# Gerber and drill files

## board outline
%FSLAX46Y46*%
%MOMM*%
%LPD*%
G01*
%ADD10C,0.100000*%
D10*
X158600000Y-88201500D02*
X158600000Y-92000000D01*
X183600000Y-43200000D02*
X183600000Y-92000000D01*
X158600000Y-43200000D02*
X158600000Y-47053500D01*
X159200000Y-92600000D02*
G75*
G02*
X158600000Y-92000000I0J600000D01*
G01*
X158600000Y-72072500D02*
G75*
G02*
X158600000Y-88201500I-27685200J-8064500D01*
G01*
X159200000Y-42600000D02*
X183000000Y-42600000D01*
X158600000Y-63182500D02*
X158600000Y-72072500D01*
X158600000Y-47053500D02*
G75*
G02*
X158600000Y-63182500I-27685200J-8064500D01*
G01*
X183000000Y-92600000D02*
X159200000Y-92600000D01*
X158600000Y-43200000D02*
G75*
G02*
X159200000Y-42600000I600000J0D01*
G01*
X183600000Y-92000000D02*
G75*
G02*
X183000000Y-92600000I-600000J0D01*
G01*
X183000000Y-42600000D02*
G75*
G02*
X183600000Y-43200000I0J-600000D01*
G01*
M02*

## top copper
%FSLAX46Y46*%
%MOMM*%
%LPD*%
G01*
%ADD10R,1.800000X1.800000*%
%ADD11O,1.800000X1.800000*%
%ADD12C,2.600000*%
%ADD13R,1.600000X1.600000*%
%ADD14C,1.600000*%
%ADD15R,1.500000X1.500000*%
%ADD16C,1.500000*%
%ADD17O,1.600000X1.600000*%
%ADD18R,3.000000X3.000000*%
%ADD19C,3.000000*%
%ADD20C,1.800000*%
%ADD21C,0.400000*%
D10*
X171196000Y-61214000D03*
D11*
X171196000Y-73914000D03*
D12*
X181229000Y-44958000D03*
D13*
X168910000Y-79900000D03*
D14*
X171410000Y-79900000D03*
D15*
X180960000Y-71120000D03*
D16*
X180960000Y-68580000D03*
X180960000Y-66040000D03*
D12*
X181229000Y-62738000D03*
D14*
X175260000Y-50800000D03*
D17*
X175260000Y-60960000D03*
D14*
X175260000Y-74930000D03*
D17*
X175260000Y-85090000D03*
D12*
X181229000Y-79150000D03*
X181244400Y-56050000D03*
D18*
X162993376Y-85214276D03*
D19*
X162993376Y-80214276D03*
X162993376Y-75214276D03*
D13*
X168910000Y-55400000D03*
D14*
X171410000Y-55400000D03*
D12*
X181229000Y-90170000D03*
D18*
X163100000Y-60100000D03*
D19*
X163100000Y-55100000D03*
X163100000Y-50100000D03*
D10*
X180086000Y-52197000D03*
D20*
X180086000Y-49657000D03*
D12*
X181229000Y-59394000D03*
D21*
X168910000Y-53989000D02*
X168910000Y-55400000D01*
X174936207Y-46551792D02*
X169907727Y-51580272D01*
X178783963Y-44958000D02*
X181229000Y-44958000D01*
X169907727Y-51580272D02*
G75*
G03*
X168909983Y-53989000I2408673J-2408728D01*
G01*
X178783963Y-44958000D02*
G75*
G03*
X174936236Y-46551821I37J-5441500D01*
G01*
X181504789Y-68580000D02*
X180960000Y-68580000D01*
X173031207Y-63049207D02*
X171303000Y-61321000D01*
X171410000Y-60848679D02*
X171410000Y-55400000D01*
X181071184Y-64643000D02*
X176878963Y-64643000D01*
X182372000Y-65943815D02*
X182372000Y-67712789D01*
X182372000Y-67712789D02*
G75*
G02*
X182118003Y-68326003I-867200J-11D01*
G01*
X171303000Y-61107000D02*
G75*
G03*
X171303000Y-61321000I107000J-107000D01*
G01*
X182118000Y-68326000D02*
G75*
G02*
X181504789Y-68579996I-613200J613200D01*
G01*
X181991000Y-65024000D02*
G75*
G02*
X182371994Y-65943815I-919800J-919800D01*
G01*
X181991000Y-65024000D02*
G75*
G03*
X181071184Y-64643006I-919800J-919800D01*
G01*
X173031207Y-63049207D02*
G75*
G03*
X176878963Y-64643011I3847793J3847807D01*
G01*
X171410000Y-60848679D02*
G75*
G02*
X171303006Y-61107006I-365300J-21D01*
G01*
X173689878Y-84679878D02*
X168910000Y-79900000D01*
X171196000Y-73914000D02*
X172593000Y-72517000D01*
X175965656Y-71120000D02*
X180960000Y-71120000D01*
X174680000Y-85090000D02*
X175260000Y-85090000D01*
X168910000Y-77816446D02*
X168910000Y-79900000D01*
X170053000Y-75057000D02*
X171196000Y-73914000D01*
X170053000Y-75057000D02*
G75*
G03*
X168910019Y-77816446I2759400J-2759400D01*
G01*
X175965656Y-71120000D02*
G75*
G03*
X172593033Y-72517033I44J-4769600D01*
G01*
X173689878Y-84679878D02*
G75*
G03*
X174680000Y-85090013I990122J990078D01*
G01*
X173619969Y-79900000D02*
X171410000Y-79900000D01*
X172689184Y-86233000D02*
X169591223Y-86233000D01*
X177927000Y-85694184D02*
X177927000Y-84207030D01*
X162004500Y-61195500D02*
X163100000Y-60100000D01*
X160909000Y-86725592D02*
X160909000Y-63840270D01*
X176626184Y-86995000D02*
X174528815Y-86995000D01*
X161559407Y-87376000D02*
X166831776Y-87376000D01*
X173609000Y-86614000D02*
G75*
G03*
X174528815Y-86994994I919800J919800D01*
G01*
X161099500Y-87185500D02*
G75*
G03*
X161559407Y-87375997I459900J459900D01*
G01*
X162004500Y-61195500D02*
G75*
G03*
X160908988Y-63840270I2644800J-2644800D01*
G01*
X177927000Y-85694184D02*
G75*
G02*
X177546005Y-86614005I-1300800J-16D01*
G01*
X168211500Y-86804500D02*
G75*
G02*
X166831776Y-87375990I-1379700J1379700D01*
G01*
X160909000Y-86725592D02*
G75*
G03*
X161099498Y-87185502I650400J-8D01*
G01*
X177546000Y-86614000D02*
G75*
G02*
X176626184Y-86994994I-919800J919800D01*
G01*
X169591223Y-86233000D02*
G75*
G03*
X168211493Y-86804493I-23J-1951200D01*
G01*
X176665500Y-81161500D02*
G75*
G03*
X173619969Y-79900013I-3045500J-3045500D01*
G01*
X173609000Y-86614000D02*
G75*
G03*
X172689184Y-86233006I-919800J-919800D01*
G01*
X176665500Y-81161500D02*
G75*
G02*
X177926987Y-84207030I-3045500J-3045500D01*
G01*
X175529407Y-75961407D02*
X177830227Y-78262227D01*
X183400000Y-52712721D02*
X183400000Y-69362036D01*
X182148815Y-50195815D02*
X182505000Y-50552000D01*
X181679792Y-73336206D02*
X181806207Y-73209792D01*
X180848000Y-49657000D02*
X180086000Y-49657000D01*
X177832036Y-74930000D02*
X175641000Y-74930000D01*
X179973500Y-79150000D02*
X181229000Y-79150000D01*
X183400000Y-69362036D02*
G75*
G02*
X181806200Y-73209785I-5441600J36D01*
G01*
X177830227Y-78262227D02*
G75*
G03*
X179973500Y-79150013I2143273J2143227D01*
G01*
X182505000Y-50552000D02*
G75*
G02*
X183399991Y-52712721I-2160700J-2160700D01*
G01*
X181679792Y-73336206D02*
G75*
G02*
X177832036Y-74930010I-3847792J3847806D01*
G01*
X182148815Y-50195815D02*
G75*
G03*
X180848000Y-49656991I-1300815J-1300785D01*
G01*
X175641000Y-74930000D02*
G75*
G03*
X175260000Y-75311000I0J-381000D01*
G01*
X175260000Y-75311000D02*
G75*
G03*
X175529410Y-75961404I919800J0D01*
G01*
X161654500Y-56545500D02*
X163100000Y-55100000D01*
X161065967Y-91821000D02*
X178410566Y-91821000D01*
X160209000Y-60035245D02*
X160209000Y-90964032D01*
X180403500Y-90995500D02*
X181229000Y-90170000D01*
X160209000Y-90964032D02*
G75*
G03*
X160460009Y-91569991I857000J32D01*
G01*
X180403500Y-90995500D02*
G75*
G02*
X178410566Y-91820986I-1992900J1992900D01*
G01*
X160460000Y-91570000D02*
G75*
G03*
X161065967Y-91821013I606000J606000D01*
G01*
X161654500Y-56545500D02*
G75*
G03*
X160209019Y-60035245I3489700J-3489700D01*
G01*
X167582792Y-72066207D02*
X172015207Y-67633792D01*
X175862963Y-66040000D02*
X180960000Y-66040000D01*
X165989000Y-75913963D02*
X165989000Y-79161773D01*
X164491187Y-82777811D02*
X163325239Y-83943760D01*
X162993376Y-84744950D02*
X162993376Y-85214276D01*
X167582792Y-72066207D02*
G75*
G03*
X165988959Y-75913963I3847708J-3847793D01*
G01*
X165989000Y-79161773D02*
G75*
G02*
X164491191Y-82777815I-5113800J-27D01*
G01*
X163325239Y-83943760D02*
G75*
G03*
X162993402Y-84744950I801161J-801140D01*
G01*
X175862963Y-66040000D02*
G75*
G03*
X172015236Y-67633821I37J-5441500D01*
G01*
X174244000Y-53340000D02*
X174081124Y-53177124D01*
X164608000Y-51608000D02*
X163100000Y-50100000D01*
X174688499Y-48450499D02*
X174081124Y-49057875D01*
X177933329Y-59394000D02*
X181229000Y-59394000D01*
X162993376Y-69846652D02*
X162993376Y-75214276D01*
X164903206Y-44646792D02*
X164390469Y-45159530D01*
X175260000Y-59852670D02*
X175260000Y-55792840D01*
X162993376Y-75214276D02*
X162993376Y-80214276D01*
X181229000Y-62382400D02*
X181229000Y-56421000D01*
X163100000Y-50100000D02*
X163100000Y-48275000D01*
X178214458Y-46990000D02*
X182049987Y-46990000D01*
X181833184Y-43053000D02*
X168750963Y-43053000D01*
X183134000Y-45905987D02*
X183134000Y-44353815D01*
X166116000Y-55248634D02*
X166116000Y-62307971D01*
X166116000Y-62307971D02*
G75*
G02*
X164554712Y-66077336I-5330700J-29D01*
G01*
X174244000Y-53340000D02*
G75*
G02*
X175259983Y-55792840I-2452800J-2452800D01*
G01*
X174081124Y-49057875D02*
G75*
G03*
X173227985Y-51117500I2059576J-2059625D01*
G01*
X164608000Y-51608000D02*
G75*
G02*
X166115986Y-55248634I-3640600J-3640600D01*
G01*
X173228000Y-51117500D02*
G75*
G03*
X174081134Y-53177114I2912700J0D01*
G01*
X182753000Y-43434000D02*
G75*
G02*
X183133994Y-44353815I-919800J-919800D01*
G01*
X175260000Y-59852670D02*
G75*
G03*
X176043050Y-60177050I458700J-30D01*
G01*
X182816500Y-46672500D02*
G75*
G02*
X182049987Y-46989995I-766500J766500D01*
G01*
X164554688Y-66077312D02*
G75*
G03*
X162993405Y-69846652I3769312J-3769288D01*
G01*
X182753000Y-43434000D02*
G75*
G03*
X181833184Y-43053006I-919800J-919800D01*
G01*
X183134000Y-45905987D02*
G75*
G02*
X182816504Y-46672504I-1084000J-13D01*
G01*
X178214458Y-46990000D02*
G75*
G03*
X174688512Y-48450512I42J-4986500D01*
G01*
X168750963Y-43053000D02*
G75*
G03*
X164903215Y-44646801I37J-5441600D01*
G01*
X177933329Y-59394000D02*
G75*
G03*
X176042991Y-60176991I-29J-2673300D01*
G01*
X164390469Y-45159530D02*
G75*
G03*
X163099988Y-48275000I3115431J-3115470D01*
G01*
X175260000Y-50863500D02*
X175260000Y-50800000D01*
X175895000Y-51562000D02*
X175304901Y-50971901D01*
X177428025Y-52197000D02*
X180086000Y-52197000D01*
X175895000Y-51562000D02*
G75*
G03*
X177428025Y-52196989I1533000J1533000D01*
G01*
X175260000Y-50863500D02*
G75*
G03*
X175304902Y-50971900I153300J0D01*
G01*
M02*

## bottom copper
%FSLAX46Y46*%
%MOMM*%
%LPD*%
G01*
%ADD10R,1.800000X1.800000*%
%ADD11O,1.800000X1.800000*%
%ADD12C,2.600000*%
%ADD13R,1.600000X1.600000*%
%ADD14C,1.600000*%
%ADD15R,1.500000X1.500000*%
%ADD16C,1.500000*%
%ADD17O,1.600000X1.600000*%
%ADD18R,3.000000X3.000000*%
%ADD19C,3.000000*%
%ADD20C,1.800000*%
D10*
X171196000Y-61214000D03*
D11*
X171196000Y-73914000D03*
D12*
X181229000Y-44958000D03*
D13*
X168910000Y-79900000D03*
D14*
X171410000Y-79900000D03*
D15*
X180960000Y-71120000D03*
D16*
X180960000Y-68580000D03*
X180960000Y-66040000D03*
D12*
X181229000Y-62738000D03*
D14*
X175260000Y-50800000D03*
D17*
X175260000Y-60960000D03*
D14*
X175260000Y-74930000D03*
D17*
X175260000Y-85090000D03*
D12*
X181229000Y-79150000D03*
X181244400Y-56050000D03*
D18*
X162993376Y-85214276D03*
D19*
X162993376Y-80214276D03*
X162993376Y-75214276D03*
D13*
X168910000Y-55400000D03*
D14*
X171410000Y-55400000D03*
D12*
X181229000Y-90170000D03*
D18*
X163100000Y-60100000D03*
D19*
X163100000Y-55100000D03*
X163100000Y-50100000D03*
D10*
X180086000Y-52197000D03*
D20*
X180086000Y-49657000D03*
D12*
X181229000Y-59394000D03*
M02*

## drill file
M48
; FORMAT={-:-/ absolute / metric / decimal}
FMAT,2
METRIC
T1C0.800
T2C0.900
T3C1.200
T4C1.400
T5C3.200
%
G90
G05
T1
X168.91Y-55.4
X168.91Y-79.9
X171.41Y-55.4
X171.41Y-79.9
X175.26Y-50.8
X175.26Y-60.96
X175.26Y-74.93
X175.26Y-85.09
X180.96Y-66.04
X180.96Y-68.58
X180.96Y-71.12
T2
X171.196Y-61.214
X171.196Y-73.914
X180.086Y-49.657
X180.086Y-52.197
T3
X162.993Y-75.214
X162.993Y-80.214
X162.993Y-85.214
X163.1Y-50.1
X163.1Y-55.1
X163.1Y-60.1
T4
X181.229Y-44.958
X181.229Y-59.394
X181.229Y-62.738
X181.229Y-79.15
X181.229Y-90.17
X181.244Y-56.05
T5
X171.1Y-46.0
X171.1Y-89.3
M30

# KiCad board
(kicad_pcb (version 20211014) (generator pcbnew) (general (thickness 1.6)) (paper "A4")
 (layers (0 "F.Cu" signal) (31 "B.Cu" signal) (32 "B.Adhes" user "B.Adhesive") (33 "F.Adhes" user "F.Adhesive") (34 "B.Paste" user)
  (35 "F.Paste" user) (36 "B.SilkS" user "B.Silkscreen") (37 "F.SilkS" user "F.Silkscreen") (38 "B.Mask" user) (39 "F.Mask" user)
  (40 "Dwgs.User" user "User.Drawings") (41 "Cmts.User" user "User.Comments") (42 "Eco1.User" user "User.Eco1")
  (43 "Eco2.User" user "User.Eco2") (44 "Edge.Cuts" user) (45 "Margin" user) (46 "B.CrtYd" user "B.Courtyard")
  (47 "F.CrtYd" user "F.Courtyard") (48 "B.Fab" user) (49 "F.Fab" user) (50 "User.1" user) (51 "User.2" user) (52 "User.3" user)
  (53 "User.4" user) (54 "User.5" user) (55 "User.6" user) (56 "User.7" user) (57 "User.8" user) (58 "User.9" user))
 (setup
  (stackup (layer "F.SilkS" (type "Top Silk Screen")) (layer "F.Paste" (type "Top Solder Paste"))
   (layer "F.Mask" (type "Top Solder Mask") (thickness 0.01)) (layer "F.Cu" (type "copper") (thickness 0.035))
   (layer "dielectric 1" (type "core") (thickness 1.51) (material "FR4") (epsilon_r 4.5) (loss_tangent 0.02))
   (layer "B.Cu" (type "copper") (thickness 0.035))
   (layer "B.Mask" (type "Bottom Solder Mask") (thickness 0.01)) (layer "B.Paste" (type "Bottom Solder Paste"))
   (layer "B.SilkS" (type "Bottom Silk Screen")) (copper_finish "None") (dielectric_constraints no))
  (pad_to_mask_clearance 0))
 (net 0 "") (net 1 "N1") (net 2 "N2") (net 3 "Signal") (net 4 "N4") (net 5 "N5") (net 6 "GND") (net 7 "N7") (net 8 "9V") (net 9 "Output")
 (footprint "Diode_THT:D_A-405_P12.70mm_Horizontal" (layer "F.Cu") (at 171.196 61.214 -90)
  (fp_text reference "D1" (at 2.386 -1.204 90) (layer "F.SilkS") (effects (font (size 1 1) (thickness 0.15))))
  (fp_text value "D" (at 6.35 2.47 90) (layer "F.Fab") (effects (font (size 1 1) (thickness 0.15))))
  (pad "1" thru_hole rect (at 0 0 270) (size 1.8 1.8) (drill 0.9) (layers *.Cu *.Mask) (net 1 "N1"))
  (pad "2" thru_hole oval (at 12.7 0 270) (size 1.8 1.8) (drill 0.9) (layers *.Cu *.Mask) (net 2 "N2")))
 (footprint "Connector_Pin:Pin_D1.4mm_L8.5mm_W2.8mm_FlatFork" (layer "F.Cu") (at 181.229 44.958)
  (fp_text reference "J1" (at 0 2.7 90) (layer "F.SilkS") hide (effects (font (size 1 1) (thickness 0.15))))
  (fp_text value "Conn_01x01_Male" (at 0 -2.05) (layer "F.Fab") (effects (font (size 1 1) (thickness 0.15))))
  (pad "1" thru_hole circle (at 0 0) (size 2.6 2.6) (drill 1.4) (layers *.Cu *.Mask) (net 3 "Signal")))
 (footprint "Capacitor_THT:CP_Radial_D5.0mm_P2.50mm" (layer "F.Cu") (at 168.91 79.9)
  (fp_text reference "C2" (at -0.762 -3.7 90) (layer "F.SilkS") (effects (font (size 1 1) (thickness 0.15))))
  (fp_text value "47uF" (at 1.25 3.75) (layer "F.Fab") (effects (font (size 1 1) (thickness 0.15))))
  (pad "1" thru_hole rect (at 0 0) (size 1.6 1.6) (drill 0.8) (layers *.Cu *.Mask) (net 2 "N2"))
  (pad "2" thru_hole circle (at 2.5 0) (size 1.6 1.6) (drill 0.8) (layers *.Cu *.Mask) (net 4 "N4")))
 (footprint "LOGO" (layer "F.Cu") (at 164.214424 67.737512 90)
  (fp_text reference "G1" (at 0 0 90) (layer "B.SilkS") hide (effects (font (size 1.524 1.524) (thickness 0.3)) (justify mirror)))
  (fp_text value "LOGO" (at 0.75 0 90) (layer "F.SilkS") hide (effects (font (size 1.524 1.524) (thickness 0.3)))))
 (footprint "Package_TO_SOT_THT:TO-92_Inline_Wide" (layer "F.Cu") (at 180.96 71.12 90)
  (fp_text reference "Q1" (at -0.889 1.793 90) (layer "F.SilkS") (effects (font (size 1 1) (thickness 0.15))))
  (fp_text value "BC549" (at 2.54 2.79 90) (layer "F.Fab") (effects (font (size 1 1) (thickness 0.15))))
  (pad "1" thru_hole rect (at 0 0 90) (size 1.5 1.5) (drill 0.8) (layers *.Cu *.Mask) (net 2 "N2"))
  (pad "2" thru_hole circle (at 2.54 0 90) (size 1.5 1.5) (drill 0.8) (layers *.Cu *.Mask) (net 1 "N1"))
  (pad "3" thru_hole circle (at 5.08 0 90) (size 1.5 1.5) (drill 0.8) (layers *.Cu *.Mask) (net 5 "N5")))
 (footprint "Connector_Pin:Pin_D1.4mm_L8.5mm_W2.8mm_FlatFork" (layer "F.Cu") (at 181.229 62.738)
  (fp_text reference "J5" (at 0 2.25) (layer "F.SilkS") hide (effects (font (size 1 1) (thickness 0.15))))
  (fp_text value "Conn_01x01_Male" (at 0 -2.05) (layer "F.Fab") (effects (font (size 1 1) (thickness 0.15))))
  (pad "1" thru_hole circle (at 0 0) (size 2.6 2.6) (drill 1.4) (layers *.Cu *.Mask) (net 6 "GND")))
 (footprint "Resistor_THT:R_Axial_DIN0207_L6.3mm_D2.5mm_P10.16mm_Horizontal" (layer "F.Cu") (at 175.26 50.8 -90)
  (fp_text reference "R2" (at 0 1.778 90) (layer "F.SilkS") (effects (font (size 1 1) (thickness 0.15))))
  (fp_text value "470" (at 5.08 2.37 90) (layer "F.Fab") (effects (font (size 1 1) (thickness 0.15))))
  (pad "1" thru_hole circle (at 0 0 270) (size 1.6 1.6) (drill 0.8) (layers *.Cu *.Mask) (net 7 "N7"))
  (pad "2" thru_hole oval (at 10.16 0 270) (size 1.6 1.6) (drill 0.8) (layers *.Cu *.Mask) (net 6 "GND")))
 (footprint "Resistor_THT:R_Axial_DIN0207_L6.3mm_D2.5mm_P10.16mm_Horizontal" (layer "F.Cu") (at 175.26 74.93 -90)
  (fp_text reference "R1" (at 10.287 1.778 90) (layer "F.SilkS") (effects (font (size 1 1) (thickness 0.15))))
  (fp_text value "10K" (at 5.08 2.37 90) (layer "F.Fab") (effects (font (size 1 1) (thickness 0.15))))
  (pad "1" thru_hole circle (at 0 0 270) (size 1.6 1.6) (drill 0.8) (layers *.Cu *.Mask) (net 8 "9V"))
  (pad "2" thru_hole oval (at 10.16 0 270) (size 1.6 1.6) (drill 0.8) (layers *.Cu *.Mask) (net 2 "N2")))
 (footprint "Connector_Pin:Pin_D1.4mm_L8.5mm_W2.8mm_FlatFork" (layer "F.Cu") (at 181.229 79.15)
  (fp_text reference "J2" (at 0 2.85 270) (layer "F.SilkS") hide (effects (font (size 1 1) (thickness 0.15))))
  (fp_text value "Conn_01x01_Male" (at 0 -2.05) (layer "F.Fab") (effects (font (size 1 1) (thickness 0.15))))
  (pad "1" thru_hole circle (at 0 0) (size 2.6 2.6) (drill 1.4) (layers *.Cu *.Mask) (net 8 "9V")))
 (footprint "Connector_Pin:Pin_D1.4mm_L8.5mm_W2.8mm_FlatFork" (layer "F.Cu") (at 181.2444 56.05)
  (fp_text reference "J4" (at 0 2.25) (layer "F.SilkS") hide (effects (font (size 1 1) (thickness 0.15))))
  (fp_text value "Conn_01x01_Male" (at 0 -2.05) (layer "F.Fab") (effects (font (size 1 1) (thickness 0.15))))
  (pad "1" thru_hole circle (at 0 0) (size 2.6 2.6) (drill 1.4) (layers *.Cu *.Mask) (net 6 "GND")))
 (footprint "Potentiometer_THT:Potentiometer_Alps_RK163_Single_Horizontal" (layer "F.Cu") (at 162.7775 79.996 180)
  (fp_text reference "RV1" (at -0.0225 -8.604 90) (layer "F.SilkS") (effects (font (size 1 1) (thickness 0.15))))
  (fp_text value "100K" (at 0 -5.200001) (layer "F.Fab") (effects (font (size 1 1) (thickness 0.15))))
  (pad "1" thru_hole rect (at -0.215876 -5.218276) (size 3 3) (drill 1.2) (layers *.Cu *.Mask) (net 5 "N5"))
  (pad "2" thru_hole circle (at -0.215876 -0.218276) (size 3 3) (drill 1.2) (layers *.Cu *.Mask) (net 6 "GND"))
  (pad "3" thru_hole circle (at -0.215876 4.781724) (size 3 3) (drill 1.2) (layers *.Cu *.Mask) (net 6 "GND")))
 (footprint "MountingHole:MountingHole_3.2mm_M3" (layer "F.Cu") (at 171.1 46)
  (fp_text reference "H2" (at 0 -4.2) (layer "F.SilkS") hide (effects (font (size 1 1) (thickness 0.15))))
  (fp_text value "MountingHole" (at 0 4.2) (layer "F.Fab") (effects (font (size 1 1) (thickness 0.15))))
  (pad "" np_thru_hole circle (at 0 0) (size 3.2 3.2) (drill 3.2) (layers *.Cu *.Mask)))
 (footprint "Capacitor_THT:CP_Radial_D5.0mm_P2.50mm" (layer "F.Cu") (at 168.91 55.4)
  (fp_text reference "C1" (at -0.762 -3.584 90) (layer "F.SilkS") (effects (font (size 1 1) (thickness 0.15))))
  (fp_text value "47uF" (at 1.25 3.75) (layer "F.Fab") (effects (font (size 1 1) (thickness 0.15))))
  (pad "1" thru_hole rect (at 0 0) (size 1.6 1.6) (drill 0.8) (layers *.Cu *.Mask) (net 3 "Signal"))
  (pad "2" thru_hole circle (at 2.5 0) (size 1.6 1.6) (drill 0.8) (layers *.Cu *.Mask) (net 1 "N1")))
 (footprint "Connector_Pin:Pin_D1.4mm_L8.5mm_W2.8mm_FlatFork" (layer "F.Cu") (at 181.229 90.17)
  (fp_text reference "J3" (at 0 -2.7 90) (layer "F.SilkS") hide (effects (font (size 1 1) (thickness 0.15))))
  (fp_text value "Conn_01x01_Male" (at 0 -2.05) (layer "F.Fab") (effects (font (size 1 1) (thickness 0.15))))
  (pad "1" thru_hole circle (at 0 0) (size 2.6 2.6) (drill 1.4) (layers *.Cu *.Mask) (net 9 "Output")))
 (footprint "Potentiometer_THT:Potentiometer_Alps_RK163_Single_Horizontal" (layer "F.Cu") (at 163.1 60.1 180)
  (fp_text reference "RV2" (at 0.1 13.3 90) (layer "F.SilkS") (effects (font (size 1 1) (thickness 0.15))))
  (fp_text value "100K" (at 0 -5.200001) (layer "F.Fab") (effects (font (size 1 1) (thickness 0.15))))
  (pad "1" thru_hole rect (at 0 0) (size 3 3) (drill 1.2) (layers *.Cu *.Mask) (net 4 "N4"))
  (pad "2" thru_hole circle (at 0 5) (size 3 3) (drill 1.2) (layers *.Cu *.Mask) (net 9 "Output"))
  (pad "3" thru_hole circle (at 0 10) (size 3 3) (drill 1.2) (layers *.Cu *.Mask) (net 6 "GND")))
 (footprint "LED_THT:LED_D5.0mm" (layer "F.Cu") (at 180.086 52.197 90)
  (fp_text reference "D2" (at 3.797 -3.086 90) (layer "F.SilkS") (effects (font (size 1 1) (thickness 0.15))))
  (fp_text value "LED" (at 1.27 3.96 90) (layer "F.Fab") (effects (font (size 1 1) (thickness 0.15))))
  (pad "1" thru_hole rect (at 0 0 90) (size 1.8 1.8) (drill 0.9) (layers *.Cu *.Mask) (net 7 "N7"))
  (pad "2" thru_hole circle (at 2.54 0 90) (size 1.8 1.8) (drill 0.9) (layers *.Cu *.Mask) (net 8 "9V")))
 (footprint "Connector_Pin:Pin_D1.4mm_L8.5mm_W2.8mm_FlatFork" (layer "F.Cu") (at 181.229 59.394 180)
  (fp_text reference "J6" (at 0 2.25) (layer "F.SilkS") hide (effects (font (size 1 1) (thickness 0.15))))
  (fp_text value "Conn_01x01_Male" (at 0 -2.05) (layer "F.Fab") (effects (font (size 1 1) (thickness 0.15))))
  (pad "1" thru_hole circle (at 0 0 180) (size 2.6 2.6) (drill 1.4) (layers *.Cu *.Mask) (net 6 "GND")))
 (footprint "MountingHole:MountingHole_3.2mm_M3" (layer "F.Cu") (at 171.1 89.3)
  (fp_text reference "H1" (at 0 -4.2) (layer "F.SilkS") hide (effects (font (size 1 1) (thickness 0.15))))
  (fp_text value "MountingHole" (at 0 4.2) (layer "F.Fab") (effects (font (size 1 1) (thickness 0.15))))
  (pad "" np_thru_hole circle (at 0 0) (size 3.2 3.2) (drill 3.2) (layers *.Cu *.Mask)))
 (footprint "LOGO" (layer "B.Cu") (at 166.470469 67.485836 -90)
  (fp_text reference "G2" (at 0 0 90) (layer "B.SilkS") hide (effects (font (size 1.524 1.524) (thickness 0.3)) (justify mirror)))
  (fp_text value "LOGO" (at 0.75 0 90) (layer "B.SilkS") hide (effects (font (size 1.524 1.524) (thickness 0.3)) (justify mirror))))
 (gr_line (start 158.6 88.2015) (end 158.6 92) (layer "Edge.Cuts") (width 0.1))
 (gr_line (start 183.6 43.2) (end 183.6 92) (layer "Edge.Cuts") (width 0.1))
 (gr_line (start 158.6 43.2) (end 158.6 47.0535) (layer "Edge.Cuts") (width 0.1))
 (gr_arc (start 159.2 92.6) (mid 158.775736 92.424264) (end 158.6 92) (layer "Edge.Cuts") (width 0.1))
 (gr_arc (start 158.6 72.0725) (mid 159.750654 80.137) (end 158.6 88.2015) (layer "Edge.Cuts") (width 0.1))
 (gr_line (start 159.2 42.6) (end 183 42.6) (layer "Edge.Cuts") (width 0.1))
 (gr_line (start 158.6 63.1825) (end 158.6 72.0725) (layer "Edge.Cuts") (width 0.1))
 (gr_arc (start 158.6 47.0535) (mid 159.750654 55.118) (end 158.6 63.1825) (layer "Edge.Cuts") (width 0.1))
 (gr_line (start 183 92.6) (end 159.2 92.6) (layer "Edge.Cuts") (width 0.1))
 (gr_arc (start 158.6 43.2) (mid 158.775736 42.775736) (end 159.2 42.6) (layer "Edge.Cuts") (width 0.1))
 (gr_arc (start 183.6 92) (mid 183.424264 92.424264) (end 183 92.6) (layer "Edge.Cuts") (width 0.1))
 (gr_arc (start 183 42.6) (mid 183.424264 42.775736) (end 183.6 43.2) (layer "Edge.Cuts") (width 0.1))
 (segment (start 168.91 53.989) (end 168.91 55.4) (width 0.4) (layer "F.Cu") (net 3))
 (segment (start 174.936207 46.551792) (end 169.907727 51.580272) (width 0.4) (layer "F.Cu") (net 3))
 (segment (start 178.783963 44.958) (end 181.229 44.958) (width 0.4) (layer "F.Cu") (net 3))
 (arc (start 169.907727 51.580272) (mid 169.1693 52.685405) (end 168.91 53.989) (width 0.4) (layer "F.Cu") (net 3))
 (arc (start 178.783963 44.958) (mid 176.701572 45.372213) (end 174.936207 46.551792) (width 0.4) (layer "F.Cu") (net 3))
 (segment (start 181.504789 68.58) (end 180.96 68.58) (width 0.4) (layer "F.Cu") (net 1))
 (segment (start 173.031207 63.049207) (end 171.303 61.321) (width 0.4) (layer "F.Cu") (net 1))
 (segment (start 171.41 60.848679) (end 171.41 55.4) (width 0.4) (layer "F.Cu") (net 1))
 (segment (start 181.071184 64.643) (end 176.878963 64.643) (width 0.4) (layer "F.Cu") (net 1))
 (segment (start 182.372 65.943815) (end 182.372 67.712789) (width 0.4) (layer "F.Cu") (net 1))
 (arc (start 182.372 67.712789) (mid 182.305987 68.044656) (end 182.118 68.326) (width 0.4) (layer "F.Cu") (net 1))
 (arc (start 171.303 61.107) (mid 171.258679 61.214) (end 171.303 61.321) (width 0.4) (layer "F.Cu") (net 1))
 (arc (start 182.118 68.326) (mid 181.836656 68.513987) (end 181.504789 68.58) (width 0.4) (layer "F.Cu") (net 1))
 (arc (start 181.991 65.024) (mid 182.272981 65.446014) (end 182.372 65.943815) (width 0.4) (layer "F.Cu") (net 1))
 (arc (start 181.991 65.024) (mid 181.568984 64.742018) (end 181.071184 64.643) (width 0.4) (layer "F.Cu") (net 1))
 (arc (start 173.031207 63.049207) (mid 174.796572 64.228786) (end 176.878963 64.643) (width 0.4) (layer "F.Cu") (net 1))
 (arc (start 171.41 60.848679) (mid 171.382191 60.988481) (end 171.303 61.107) (width 0.4) (layer "F.Cu") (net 1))
 (segment (start 173.689878 84.679878) (end 168.91 79.9) (width 0.4) (layer "F.Cu") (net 2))
 (segment (start 171.196 73.914) (end 172.593 72.517) (width 0.4) (layer "F.Cu") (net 2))
 (segment (start 175.965656 71.12) (end 180.96 71.12) (width 0.4) (layer "F.Cu") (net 2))
 (segment (start 174.68 85.09) (end 175.26 85.09) (width 0.4) (layer "F.Cu") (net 2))
 (segment (start 168.91 77.816446) (end 168.91 79.9) (width 0.4) (layer "F.Cu") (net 2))
 (segment (start 170.053 75.057) (end 171.196 73.914) (width 0.4) (layer "F.Cu") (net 2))
 (arc (start 170.053 75.057) (mid 169.207056 76.323044) (end 168.91 77.816446) (width 0.4) (layer "F.Cu") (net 2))
 (arc (start 175.965656 71.12) (mid 174.140387 71.483068) (end 172.593 72.517) (width 0.4) (layer "F.Cu") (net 2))
 (arc (start 173.689878 84.679878) (mid 174.144149 84.983412) (end 174.68 85.09) (width 0.4) (layer "F.Cu") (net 2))
 (segment (start 173.619969 79.9) (end 171.41 79.9) (width 0.4) (layer "F.Cu") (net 4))
 (segment (start 172.689184 86.233) (end 169.591223 86.233) (width 0.4) (layer "F.Cu") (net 4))
 (segment (start 177.927 85.694184) (end 177.927 84.20703) (width 0.4) (layer "F.Cu") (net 4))
 (segment (start 162.0045 61.1955) (end 163.1 60.1) (width 0.4) (layer "F.Cu") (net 4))
 (segment (start 160.909 86.725592) (end 160.909 63.84027) (width 0.4) (layer "F.Cu") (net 4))
 (segment (start 176.626184 86.995) (end 174.528815 86.995) (width 0.4) (layer "F.Cu") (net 4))
 (segment (start 161.559407 87.376) (end 166.831776 87.376) (width 0.4) (layer "F.Cu") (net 4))
 (arc (start 173.609 86.614) (mid 174.031014 86.895981) (end 174.528815 86.995) (width 0.4) (layer "F.Cu") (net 4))
 (arc (start 161.0995 87.1855) (mid 161.310507 87.32649) (end 161.559407 87.376) (width 0.4) (layer "F.Cu") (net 4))
 (arc (start 162.0045 61.1955) (mid 161.193711 62.40893) (end 160.909 63.84027) (width 0.4) (layer "F.Cu") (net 4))
 (arc (start 177.927 85.694184) (mid 177.827981 86.191984) (end 177.546 86.614) (width 0.4) (layer "F.Cu") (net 4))
 (arc (start 168.2115 86.8045) (mid 167.578477 87.227471) (end 166.831776 87.376) (width 0.4) (layer "F.Cu") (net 4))
 (arc (start 160.909 86.725592) (mid 160.958509 86.974492) (end 161.0995 87.1855) (width 0.4) (layer "F.Cu") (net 4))
 (arc (start 177.546 86.614) (mid 177.123984 86.895981) (end 176.626184 86.995) (width 0.4) (layer "F.Cu") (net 4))
 (arc (start 169.591223 86.233) (mid 168.844522 86.381528) (end 168.2115 86.8045) (width 0.4) (layer "F.Cu") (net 4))
 (arc (start 176.6655 81.1615) (mid 175.268198 80.227853) (end 173.619969 79.9) (width 0.4) (layer "F.Cu") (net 4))
 (arc (start 173.609 86.614) (mid 173.186984 86.332018) (end 172.689184 86.233) (width 0.4) (layer "F.Cu") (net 4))
 (arc (start 176.6655 81.1615) (mid 177.599146 82.558801) (end 177.927 84.20703) (width 0.4) (layer "F.Cu") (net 4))
 (segment (start 175.529407 75.961407) (end 177.830227 78.262227) (width 0.4) (layer "F.Cu") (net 8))
 (segment (start 183.4 52.712721) (end 183.4 69.362036) (width 0.4) (layer "F.Cu") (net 8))
 (segment (start 182.148815 50.195815) (end 182.505 50.552) (width 0.4) (layer "F.Cu") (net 8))
 (segment (start 181.679792 73.336206) (end 181.806207 73.209792) (width 0.4) (layer "F.Cu") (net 8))
 (segment (start 180.848 49.657) (end 180.086 49.657) (width 0.4) (layer "F.Cu") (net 8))
 (segment (start 177.832036 74.93) (end 175.641 74.93) (width 0.4) (layer "F.Cu") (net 8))
 (segment (start 179.9735 79.15) (end 181.229 79.15) (width 0.4) (layer "F.Cu") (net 8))
 (arc (start 183.4 69.362036) (mid 182.985786 71.444426) (end 181.806207 73.209792) (width 0.4) (layer "F.Cu") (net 8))
 (arc (start 177.830227 78.262227) (mid 178.813569 78.919275) (end 179.9735 79.15) (width 0.4) (layer "F.Cu") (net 8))
 (arc (start 182.505 50.552) (mid 183.167397 51.543347) (end 183.4 52.712721) (width 0.4) (layer "F.Cu") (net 8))
 (arc (start 181.679792 73.336206) (mid 179.914426 74.515786) (end 177.832036 74.93) (width 0.4) (layer "F.Cu") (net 8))
 (arc (start 182.148815 50.195815) (mid 181.551996 49.797033) (end 180.848 49.657) (width 0.4) (layer "F.Cu") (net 8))
 (arc (start 175.641 74.93) (mid 175.371592 75.041592) (end 175.26 75.311) (width 0.4) (layer "F.Cu") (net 8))
 (arc (start 175.26 75.311) (mid 175.330016 75.662997) (end 175.529407 75.961407) (width 0.4) (layer "F.Cu") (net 8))
 (segment (start 161.6545 56.5455) (end 163.1 55.1) (width 0.4) (layer "F.Cu") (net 9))
 (segment (start 161.065967 91.821) (end 178.410566 91.821) (width 0.4) (layer "F.Cu") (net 9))
 (segment (start 160.209 60.035245) (end 160.209 90.964032) (width 0.4) (layer "F.Cu") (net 9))
 (segment (start 180.4035 90.9955) (end 181.229 90.17) (width 0.4) (layer "F.Cu") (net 9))
 (arc (start 160.209 90.964032) (mid 160.274232 91.291979) (end 160.46 91.57) (width 0.4) (layer "F.Cu") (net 9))
 (arc (start 180.4035 90.9955) (mid 179.489134 91.606459) (end 178.410566 91.821) (width 0.4) (layer "F.Cu") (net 9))
 (arc (start 160.46 91.57) (mid 160.73802 91.755767) (end 161.065967 91.821) (width 0.4) (layer "F.Cu") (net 9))
 (arc (start 161.6545 56.5455) (mid 160.584673 58.146608) (end 160.209 60.035245) (width 0.4) (layer "F.Cu") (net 9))
 (segment (start 167.582792 72.066207) (end 172.015207 67.633792) (width 0.4) (layer "F.Cu") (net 5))
 (segment (start 175.862963 66.04) (end 180.96 66.04) (width 0.4) (layer "F.Cu") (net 5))
 (segment (start 165.989 75.913963) (end 165.989 79.161773) (width 0.4) (layer "F.Cu") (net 5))
 (segment (start 164.491187 82.777811) (end 163.325239 83.94376) (width 0.4) (layer "F.Cu") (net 5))
 (segment (start 162.993376 84.74495) (end 162.993376 85.214276) (width 0.4) (layer "F.Cu") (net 5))
 (arc (start 167.582792 72.066207) (mid 166.403213 73.831572) (end 165.989 75.913963) (width 0.4) (layer "F.Cu") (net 5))
 (arc (start 165.989 79.161773) (mid 165.599731 81.118759) (end 164.491187 82.777811) (width 0.4) (layer "F.Cu") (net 5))
 (arc (start 163.325239 83.94376) (mid 163.079624 84.311349) (end 162.993376 84.74495) (width 0.4) (layer "F.Cu") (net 5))
 (arc (start 175.862963 66.04) (mid 173.780572 66.454213) (end 172.015207 67.633792) (width 0.4) (layer "F.Cu") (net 5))
 (segment (start 174.244 53.34) (end 174.081124 53.177124) (width 0.4) (layer "F.Cu") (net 6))
 (segment (start 164.608 51.608) (end 163.1 50.1) (width 0.4) (layer "F.Cu") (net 6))
 (segment (start 174.688499 48.450499) (end 174.081124 49.057875) (width 0.4) (layer "F.Cu") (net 6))
 (segment (start 177.933329 59.394) (end 181.229 59.394) (width 0.4) (layer "F.Cu") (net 6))
 (segment (start 162.993376 69.846652) (end 162.993376 75.214276) (width 0.4) (layer "F.Cu") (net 6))
 (segment (start 164.903206 44.646792) (end 164.390469 45.15953) (width 0.4) (layer "F.Cu") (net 6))
 (segment (start 175.26 59.85267) (end 175.26 55.79284) (width 0.4) (layer "F.Cu") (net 6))
 (segment (start 162.993376 75.214276) (end 162.993376 80.214276) (width 0.4) (layer "F.Cu") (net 6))
 (segment (start 181.229 62.3824) (end 181.229 56.421) (width 0.4) (layer "F.Cu") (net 6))
 (segment (start 163.1 50.1) (end 163.1 48.275) (width 0.4) (layer "F.Cu") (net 6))
 (segment (start 178.214458 46.99) (end 182.049987 46.99) (width 0.4) (layer "F.Cu") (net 6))
 (segment (start 181.833184 43.053) (end 168.750963 43.053) (width 0.4) (layer "F.Cu") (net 6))
 (segment (start 183.134 45.905987) (end 183.134 44.353815) (width 0.4) (layer "F.Cu") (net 6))
 (segment (start 166.116 55.248634) (end 166.116 62.307971) (width 0.4) (layer "F.Cu") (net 6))
 (arc (start 166.116 62.307971) (mid 165.710228 64.347923) (end 164.554688 66.077312) (width 0.4) (layer "F.Cu") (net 6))
 (arc (start 174.244 53.34) (mid 174.99595 54.465372) (end 175.26 55.79284) (width 0.4) (layer "F.Cu") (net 6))
 (arc (start 174.081124 49.057875) (mid 173.449719 50.002839) (end 173.228 51.1175) (width 0.4) (layer "F.Cu") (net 6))
 (arc (start 164.608 51.608) (mid 165.724083 53.278337) (end 166.116 55.248634) (width 0.4) (layer "F.Cu") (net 6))
 (arc (start 173.228 51.1175) (mid 173.449719 52.23216) (end 174.081124 53.177124) (width 0.4) (layer "F.Cu") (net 6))
 (arc (start 182.753 43.434) (mid 183.034981 43.856014) (end 183.134 44.353815) (width 0.4) (layer "F.Cu") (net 6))
 (arc (start 175.26 59.85267) (mid 175.543145 60.276427) (end 176.043 60.177) (width 0.4) (layer "F.Cu") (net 6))
 (arc (start 182.8165 46.6725) (mid 182.46482 46.907484) (end 182.049987 46.99) (width 0.4) (layer "F.Cu") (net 6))
 (arc (start 164.554688 66.077312) (mid 163.399147 67.8067) (end 162.993376 69.846652) (width 0.4) (layer "F.Cu") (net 6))
 (arc (start 182.753 43.434) (mid 182.330984 43.152018) (end 181.833184 43.053) (width 0.4) (layer "F.Cu") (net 6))
 (arc (start 183.134 45.905987) (mid 183.051484 46.32082) (end 182.8165 46.6725) (width 0.4) (layer "F.Cu") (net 6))
 (arc (start 178.214458 46.99) (mid 176.306223 47.369571) (end 174.688499 48.450499) (width 0.4) (layer "F.Cu") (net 6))
 (arc (start 168.750963 43.053) (mid 166.668572 43.467213) (end 164.903206 44.646792) (width 0.4) (layer "F.Cu") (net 6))
 (arc (start 177.933329 59.394) (mid 176.91029 59.597495) (end 176.043 60.177) (width 0.4) (layer "F.Cu") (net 6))
 (arc (start 164.390469 45.15953) (mid 163.435381 46.588919) (end 163.1 48.275) (width 0.4) (layer "F.Cu") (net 6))
 (segment (start 175.26 50.8635) (end 175.26 50.8) (width 0.4) (layer "F.Cu") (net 7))
 (segment (start 175.895 51.562) (end 175.304901 50.971901) (width 0.4) (layer "F.Cu") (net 7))
 (segment (start 177.428025 52.197) (end 180.086 52.197) (width 0.4) (layer "F.Cu") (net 7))
 (arc (start 175.895 51.562) (mid 176.598357 52.031968) (end 177.428025 52.197) (width 0.4) (layer "F.Cu") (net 7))
 (arc (start 175.26 50.8635) (mid 175.271669 50.922166) (end 175.304901 50.971901) (width 0.4) (layer "F.Cu") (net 7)))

